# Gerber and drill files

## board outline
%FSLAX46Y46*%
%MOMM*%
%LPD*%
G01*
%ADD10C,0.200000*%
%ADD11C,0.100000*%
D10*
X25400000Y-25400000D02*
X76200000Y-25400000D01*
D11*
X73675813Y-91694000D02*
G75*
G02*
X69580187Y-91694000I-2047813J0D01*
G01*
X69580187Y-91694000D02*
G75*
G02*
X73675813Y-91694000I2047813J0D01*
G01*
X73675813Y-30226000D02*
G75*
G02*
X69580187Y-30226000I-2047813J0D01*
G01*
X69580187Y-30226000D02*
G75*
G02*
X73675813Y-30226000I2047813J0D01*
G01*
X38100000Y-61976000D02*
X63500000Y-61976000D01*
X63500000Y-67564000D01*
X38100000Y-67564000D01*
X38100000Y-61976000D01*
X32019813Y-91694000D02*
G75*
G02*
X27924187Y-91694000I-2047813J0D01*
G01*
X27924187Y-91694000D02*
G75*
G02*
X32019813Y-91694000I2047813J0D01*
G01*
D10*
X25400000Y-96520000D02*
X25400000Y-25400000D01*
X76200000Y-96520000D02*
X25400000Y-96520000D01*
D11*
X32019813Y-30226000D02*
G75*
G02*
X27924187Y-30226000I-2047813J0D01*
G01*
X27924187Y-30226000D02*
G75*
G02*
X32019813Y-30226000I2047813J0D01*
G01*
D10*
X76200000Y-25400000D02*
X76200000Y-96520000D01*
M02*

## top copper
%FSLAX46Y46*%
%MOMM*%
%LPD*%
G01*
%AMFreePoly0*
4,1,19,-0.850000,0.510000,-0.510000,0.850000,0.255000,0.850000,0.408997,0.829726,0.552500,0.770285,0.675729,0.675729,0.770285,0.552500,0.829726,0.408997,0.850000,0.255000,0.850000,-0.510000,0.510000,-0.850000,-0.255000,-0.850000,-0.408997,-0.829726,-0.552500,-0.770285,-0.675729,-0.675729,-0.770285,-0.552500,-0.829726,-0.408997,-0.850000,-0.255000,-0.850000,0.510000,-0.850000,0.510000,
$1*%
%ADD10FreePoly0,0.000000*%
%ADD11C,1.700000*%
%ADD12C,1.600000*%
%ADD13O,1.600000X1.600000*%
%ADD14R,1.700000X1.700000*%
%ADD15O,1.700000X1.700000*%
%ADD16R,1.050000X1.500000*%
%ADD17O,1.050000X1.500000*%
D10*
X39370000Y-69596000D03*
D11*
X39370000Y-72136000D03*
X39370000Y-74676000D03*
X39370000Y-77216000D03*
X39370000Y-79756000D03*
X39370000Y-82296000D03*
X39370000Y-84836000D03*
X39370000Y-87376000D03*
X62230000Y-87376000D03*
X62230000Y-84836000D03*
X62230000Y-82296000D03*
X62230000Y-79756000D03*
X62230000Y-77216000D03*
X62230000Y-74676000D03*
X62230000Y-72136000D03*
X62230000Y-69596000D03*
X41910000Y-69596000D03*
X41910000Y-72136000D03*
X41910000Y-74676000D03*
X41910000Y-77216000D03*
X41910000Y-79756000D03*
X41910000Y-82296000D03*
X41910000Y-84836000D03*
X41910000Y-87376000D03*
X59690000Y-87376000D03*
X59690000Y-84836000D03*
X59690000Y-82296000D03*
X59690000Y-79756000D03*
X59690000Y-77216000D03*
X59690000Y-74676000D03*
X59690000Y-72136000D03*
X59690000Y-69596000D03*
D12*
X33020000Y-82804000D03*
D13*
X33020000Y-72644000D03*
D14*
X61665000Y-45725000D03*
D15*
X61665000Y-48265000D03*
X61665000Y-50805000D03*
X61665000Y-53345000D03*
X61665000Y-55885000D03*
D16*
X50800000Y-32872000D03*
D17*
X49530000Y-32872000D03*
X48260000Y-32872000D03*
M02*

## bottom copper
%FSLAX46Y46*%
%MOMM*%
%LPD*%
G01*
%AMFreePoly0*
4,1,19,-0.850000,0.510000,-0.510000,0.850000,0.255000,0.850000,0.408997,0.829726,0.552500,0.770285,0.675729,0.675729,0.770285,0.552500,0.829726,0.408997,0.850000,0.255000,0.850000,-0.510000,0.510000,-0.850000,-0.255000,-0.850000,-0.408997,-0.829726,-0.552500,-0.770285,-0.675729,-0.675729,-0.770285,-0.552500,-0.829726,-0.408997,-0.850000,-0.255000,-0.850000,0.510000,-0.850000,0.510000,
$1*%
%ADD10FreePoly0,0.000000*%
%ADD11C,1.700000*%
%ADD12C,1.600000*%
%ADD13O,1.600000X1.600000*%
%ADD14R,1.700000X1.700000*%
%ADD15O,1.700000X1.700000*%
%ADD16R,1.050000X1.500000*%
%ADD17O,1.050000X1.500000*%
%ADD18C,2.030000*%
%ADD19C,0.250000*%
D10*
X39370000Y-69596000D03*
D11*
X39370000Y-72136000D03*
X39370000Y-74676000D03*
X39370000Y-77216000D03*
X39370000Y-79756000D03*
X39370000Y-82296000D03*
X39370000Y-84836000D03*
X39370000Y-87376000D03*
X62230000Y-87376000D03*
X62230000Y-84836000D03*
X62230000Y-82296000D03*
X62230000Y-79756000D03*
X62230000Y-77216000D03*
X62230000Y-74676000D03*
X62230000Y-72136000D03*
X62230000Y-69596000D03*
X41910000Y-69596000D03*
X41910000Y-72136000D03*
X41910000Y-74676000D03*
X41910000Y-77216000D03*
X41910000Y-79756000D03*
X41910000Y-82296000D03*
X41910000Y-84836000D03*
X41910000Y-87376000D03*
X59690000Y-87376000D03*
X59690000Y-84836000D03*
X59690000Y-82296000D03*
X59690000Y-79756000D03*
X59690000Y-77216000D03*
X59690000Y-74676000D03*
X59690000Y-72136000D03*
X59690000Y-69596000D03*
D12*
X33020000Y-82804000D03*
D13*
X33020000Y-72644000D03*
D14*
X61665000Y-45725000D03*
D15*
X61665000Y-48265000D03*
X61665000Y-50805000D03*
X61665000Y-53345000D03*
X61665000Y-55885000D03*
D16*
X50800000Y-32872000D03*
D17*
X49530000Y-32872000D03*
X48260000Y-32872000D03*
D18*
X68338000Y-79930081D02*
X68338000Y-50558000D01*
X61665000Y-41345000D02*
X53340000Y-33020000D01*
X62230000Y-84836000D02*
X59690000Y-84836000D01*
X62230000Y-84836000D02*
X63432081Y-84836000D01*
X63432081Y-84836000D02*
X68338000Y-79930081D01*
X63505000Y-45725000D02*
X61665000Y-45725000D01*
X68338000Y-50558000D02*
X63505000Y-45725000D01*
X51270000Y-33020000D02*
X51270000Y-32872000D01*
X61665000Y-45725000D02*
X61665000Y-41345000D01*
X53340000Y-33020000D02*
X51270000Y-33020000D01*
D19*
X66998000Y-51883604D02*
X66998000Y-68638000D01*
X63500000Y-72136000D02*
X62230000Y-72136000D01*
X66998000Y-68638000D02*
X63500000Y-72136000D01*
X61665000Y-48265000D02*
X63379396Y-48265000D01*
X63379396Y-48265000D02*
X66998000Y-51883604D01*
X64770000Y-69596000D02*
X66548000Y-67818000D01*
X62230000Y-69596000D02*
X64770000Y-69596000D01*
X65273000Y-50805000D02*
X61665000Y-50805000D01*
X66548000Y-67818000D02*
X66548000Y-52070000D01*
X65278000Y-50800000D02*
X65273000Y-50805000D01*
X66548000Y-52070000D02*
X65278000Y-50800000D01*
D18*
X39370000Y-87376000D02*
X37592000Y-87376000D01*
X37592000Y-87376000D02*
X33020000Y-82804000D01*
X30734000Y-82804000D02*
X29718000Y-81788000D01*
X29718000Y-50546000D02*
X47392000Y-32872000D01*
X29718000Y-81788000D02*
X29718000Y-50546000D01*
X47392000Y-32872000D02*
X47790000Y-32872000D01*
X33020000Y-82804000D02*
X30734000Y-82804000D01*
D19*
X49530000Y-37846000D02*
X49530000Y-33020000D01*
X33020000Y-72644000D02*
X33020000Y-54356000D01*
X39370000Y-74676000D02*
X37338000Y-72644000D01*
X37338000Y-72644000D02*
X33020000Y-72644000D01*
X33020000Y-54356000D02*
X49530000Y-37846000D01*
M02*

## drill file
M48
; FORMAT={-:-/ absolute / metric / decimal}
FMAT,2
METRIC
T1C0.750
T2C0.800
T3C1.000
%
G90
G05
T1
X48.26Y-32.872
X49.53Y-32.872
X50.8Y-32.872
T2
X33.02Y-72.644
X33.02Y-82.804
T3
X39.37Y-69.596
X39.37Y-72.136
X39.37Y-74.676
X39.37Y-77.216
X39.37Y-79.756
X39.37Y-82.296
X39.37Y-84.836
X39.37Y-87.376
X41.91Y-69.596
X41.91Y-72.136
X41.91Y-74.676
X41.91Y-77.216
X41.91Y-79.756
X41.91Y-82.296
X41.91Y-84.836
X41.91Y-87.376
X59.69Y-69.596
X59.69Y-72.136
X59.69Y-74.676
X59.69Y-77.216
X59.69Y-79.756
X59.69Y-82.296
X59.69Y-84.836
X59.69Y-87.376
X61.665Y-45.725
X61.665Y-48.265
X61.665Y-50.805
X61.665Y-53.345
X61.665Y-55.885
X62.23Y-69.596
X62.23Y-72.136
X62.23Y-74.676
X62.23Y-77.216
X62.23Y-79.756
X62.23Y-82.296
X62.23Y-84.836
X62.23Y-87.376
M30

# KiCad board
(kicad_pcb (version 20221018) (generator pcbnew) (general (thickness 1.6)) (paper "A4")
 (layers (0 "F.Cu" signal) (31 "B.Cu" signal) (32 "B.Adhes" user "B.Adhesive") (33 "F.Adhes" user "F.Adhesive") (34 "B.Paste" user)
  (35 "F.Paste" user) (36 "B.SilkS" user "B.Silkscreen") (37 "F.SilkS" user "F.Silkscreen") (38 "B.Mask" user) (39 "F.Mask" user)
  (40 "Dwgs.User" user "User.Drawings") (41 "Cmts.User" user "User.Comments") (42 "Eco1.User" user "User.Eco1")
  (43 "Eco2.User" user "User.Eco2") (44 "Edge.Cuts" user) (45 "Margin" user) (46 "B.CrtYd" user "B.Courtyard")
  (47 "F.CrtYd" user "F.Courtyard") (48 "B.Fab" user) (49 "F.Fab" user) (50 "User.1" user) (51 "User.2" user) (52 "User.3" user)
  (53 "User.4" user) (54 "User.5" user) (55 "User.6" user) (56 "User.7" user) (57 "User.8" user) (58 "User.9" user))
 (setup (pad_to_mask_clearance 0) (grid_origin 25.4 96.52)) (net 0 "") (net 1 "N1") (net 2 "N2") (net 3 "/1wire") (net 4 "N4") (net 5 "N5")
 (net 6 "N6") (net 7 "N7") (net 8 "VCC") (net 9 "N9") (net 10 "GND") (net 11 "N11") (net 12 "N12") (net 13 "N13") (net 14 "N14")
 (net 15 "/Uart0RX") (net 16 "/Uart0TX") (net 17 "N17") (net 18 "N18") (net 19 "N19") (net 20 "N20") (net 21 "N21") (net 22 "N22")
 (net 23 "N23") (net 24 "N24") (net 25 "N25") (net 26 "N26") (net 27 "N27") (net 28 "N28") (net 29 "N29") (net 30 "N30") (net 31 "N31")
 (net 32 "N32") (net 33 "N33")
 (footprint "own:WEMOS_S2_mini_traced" (layer "F.Cu") (at 39.37 69.596)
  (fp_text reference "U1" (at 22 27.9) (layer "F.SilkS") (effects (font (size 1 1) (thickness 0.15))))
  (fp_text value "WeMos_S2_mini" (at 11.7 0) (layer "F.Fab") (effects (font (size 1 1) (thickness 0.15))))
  (pad "1" thru_hole roundrect (at 0 0) (size 1.7 1.7) (drill 1) (layers "*.Cu" "*.Mask") (roundrect_rratio 0.35) (chamfer_ratio 0.2)
   (chamfer top_left bottom_right) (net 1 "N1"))
  (pad "2" thru_hole circle (at 0 2.54) (size 1.7 1.7) (drill 1) (layers "*.Cu" "*.Mask") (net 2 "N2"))
  (pad "3" thru_hole circle (at 0 5.08) (size 1.7 1.7) (drill 1) (layers "*.Cu" "*.Mask") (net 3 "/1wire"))
  (pad "4" thru_hole circle (at 0 7.62) (size 1.7 1.7) (drill 1) (layers "*.Cu" "*.Mask") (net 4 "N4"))
  (pad "5" thru_hole circle (at 0 10.16) (size 1.7 1.7) (drill 1) (layers "*.Cu" "*.Mask") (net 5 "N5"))
  (pad "6" thru_hole circle (at 0 12.7) (size 1.7 1.7) (drill 1) (layers "*.Cu" "*.Mask") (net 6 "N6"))
  (pad "7" thru_hole circle (at 0 15.24) (size 1.7 1.7) (drill 1) (layers "*.Cu" "*.Mask") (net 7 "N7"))
  (pad "8" thru_hole circle (at 0 17.78) (size 1.7 1.7) (drill 1) (layers "*.Cu" "*.Mask") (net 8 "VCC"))
  (pad "9" thru_hole circle (at 22.86 17.78) (size 1.7 1.7) (drill 1) (layers "*.Cu" "*.Mask") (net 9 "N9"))
  (pad "10" thru_hole circle (at 22.86 15.24) (size 1.7 1.7) (drill 1) (layers "*.Cu" "*.Mask") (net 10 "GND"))
  (pad "11" thru_hole circle (at 22.86 12.7) (size 1.7 1.7) (drill 1) (layers "*.Cu" "*.Mask") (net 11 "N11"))
  (pad "12" thru_hole circle (at 22.86 10.16) (size 1.7 1.7) (drill 1) (layers "*.Cu" "*.Mask") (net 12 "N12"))
  (pad "13" thru_hole circle (at 22.86 7.62) (size 1.7 1.7) (drill 1) (layers "*.Cu" "*.Mask") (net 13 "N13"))
  (pad "14" thru_hole circle (at 22.86 5.08) (size 1.7 1.7) (drill 1) (layers "*.Cu" "*.Mask") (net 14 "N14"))
  (pad "15" thru_hole circle (at 22.86 2.54) (size 1.7 1.7) (drill 1) (layers "*.Cu" "*.Mask") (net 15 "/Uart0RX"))
  (pad "16" thru_hole circle (at 22.86 0) (size 1.7 1.7) (drill 1) (layers "*.Cu" "*.Mask") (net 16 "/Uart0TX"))
  (pad "17" thru_hole circle (at 2.54 0) (size 1.7 1.7) (drill 1) (layers "*.Cu" "*.Mask") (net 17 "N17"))
  (pad "18" thru_hole circle (at 2.54 2.54) (size 1.7 1.7) (drill 1) (layers "*.Cu" "*.Mask") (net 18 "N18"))
  (pad "19" thru_hole circle (at 2.54 5.08) (size 1.7 1.7) (drill 1) (layers "*.Cu" "*.Mask") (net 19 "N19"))
  (pad "20" thru_hole circle (at 2.54 7.62) (size 1.7 1.7) (drill 1) (layers "*.Cu" "*.Mask") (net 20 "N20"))
  (pad "21" thru_hole circle (at 2.54 10.16) (size 1.7 1.7) (drill 1) (layers "*.Cu" "*.Mask") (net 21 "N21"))
  (pad "22" thru_hole circle (at 2.54 12.7) (size 1.7 1.7) (drill 1) (layers "*.Cu" "*.Mask") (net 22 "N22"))
  (pad "23" thru_hole circle (at 2.54 15.24) (size 1.7 1.7) (drill 1) (layers "*.Cu" "*.Mask") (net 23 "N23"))
  (pad "24" thru_hole circle (at 2.54 17.78) (size 1.7 1.7) (drill 1) (layers "*.Cu" "*.Mask") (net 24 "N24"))
  (pad "25" thru_hole circle (at 20.32 17.78) (size 1.7 1.7) (drill 1) (layers "*.Cu" "*.Mask") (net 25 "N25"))
  (pad "26" thru_hole circle (at 20.32 15.24) (size 1.7 1.7) (drill 1) (layers "*.Cu" "*.Mask") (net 10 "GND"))
  (pad "27" thru_hole circle (at 20.32 12.7) (size 1.7 1.7) (drill 1) (layers "*.Cu" "*.Mask") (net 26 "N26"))
  (pad "28" thru_hole circle (at 20.32 10.16) (size 1.7 1.7) (drill 1) (layers "*.Cu" "*.Mask") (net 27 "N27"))
  (pad "29" thru_hole circle (at 20.32 7.62) (size 1.7 1.7) (drill 1) (layers "*.Cu" "*.Mask") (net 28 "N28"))
  (pad "30" thru_hole circle (at 20.32 5.08) (size 1.7 1.7) (drill 1) (layers "*.Cu" "*.Mask") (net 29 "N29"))
  (pad "31" thru_hole circle (at 20.32 2.54) (size 1.7 1.7) (drill 1) (layers "*.Cu" "*.Mask") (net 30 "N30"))
  (pad "32" thru_hole circle (at 20.32 0) (size 1.7 1.7) (drill 1) (layers "*.Cu" "*.Mask") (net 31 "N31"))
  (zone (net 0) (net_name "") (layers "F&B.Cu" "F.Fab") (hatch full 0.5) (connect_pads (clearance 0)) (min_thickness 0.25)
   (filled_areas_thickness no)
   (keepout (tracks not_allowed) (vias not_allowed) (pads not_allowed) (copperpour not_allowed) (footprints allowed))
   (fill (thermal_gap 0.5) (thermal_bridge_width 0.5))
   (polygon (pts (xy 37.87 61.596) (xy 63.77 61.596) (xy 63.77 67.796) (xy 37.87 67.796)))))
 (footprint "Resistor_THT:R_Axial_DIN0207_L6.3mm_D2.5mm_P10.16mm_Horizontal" (layer "F.Cu") (at 33.02 82.804 90)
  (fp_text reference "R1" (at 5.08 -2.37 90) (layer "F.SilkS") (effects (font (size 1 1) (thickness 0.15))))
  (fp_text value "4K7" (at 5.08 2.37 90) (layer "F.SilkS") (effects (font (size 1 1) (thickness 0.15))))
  (pad "1" thru_hole circle (at 0 0 90) (size 1.6 1.6) (drill 0.8) (layers "*.Cu" "*.Mask") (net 8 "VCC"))
  (pad "2" thru_hole oval (at 10.16 0 90) (size 1.6 1.6) (drill 0.8) (layers "*.Cu" "*.Mask") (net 3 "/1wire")))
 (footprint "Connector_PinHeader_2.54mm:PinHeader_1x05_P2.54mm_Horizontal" (layer "F.Cu") (at 61.665 45.725)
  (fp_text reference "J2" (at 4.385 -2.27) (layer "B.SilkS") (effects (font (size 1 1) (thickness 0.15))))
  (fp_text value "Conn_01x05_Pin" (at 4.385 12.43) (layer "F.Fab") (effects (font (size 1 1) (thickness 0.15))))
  (pad "1" thru_hole rect (at 0 0) (size 1.7 1.7) (drill 1) (layers "*.Cu" "*.Mask") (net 10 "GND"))
  (pad "2" thru_hole oval (at 0 2.54) (size 1.7 1.7) (drill 1) (layers "*.Cu" "*.Mask") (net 15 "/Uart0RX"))
  (pad "3" thru_hole oval (at 0 5.08) (size 1.7 1.7) (drill 1) (layers "*.Cu" "*.Mask") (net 16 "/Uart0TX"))
  (pad "4" thru_hole oval (at 0 7.62) (size 1.7 1.7) (drill 1) (layers "*.Cu" "*.Mask") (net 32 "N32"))
  (pad "5" thru_hole oval (at 0 10.16) (size 1.7 1.7) (drill 1) (layers "*.Cu" "*.Mask") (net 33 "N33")))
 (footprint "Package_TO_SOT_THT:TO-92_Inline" (layer "B.Cu") (at 50.8 32.872 180)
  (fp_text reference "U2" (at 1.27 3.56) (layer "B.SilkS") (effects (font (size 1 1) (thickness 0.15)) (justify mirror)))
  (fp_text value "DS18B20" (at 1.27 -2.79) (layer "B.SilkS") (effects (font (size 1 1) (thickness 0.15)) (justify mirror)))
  (pad "1" thru_hole rect (at 0 0 180) (size 1.05 1.5) (drill 0.75) (layers "*.Cu" "*.Mask") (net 10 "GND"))
  (pad "2" thru_hole oval (at 1.27 0 180) (size 1.05 1.5) (drill 0.75) (layers "*.Cu" "*.Mask") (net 3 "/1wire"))
  (pad "3" thru_hole oval (at 2.54 0 180) (size 1.05 1.5) (drill 0.75) (layers "*.Cu" "*.Mask") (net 8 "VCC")))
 (gr_line (start 25.4 25.4) (end 76.2 25.4) (stroke (width 0.2) (type default)) (layer "Edge.Cuts"))
 (gr_circle (center 71.628 91.694) (end 72.644 93.472) (stroke (width 0.1) (type default)) (fill none) (layer "Edge.Cuts"))
 (gr_circle (center 71.628 30.226) (end 72.644 32.004) (stroke (width 0.1) (type default)) (fill none) (layer "Edge.Cuts"))
 (gr_rect (start 38.1 61.976) (end 63.5 67.564) (stroke (width 0.1) (type default)) (fill none) (layer "Edge.Cuts"))
 (gr_circle (center 29.972 91.694) (end 30.988 93.472) (stroke (width 0.1) (type default)) (fill none) (layer "Edge.Cuts"))
 (gr_line (start 25.4 96.52) (end 25.4 25.4) (stroke (width 0.2) (type default)) (layer "Edge.Cuts"))
 (gr_line (start 76.2 96.52) (end 25.4 96.52) (stroke (width 0.2) (type default)) (layer "Edge.Cuts"))
 (gr_circle (center 29.972 30.226) (end 30.988 32.004) (stroke (width 0.1) (type default)) (fill none) (layer "Edge.Cuts"))
 (gr_line (start 76.2 25.4) (end 76.2 96.52) (stroke (width 0.2) (type default)) (layer "Edge.Cuts"))
 (segment (start 68.338 79.930081) (end 68.338 50.558) (width 2.03) (layer "B.Cu") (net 10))
 (segment (start 61.665 41.345) (end 53.34 33.02) (width 2.03) (layer "B.Cu") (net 10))
 (segment (start 62.23 84.836) (end 59.69 84.836) (width 2.03) (layer "B.Cu") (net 10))
 (segment (start 62.23 84.836) (end 63.432081 84.836) (width 2.03) (layer "B.Cu") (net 10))
 (segment (start 63.432081 84.836) (end 68.338 79.930081) (width 2.03) (layer "B.Cu") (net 10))
 (segment (start 63.505 45.725) (end 61.665 45.725) (width 2.03) (layer "B.Cu") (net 10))
 (segment (start 68.338 50.558) (end 63.505 45.725) (width 2.03) (layer "B.Cu") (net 10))
 (segment (start 51.27 33.02) (end 51.27 32.872) (width 2.03) (layer "B.Cu") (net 10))
 (segment (start 61.665 45.725) (end 61.665 41.345) (width 2.03) (layer "B.Cu") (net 10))
 (segment (start 53.34 33.02) (end 51.27 33.02) (width 2.03) (layer "B.Cu") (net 10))
 (segment (start 66.998 51.883604) (end 66.998 68.638) (width 0.25) (layer "B.Cu") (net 15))
 (segment (start 63.5 72.136) (end 62.23 72.136) (width 0.25) (layer "B.Cu") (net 15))
 (segment (start 66.998 68.638) (end 63.5 72.136) (width 0.25) (layer "B.Cu") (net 15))
 (segment (start 61.665 48.265) (end 63.379396 48.265) (width 0.25) (layer "B.Cu") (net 15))
 (segment (start 63.379396 48.265) (end 66.998 51.883604) (width 0.25) (layer "B.Cu") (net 15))
 (segment (start 64.77 69.596) (end 66.548 67.818) (width 0.25) (layer "B.Cu") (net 16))
 (segment (start 62.23 69.596) (end 64.77 69.596) (width 0.25) (layer "B.Cu") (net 16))
 (segment (start 65.273 50.805) (end 61.665 50.805) (width 0.25) (layer "B.Cu") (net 16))
 (segment (start 66.548 67.818) (end 66.548 52.07) (width 0.25) (layer "B.Cu") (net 16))
 (segment (start 65.278 50.8) (end 65.273 50.805) (width 0.25) (layer "B.Cu") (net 16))
 (segment (start 66.548 52.07) (end 65.278 50.8) (width 0.25) (layer "B.Cu") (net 16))
 (segment (start 39.37 87.376) (end 37.592 87.376) (width 2.03) (layer "B.Cu") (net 8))
 (segment (start 37.592 87.376) (end 33.02 82.804) (width 2.03) (layer "B.Cu") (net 8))
 (segment (start 30.734 82.804) (end 29.718 81.788) (width 2.03) (layer "B.Cu") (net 8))
 (segment (start 29.718 50.546) (end 47.392 32.872) (width 2.03) (layer "B.Cu") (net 8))
 (segment (start 29.718 81.788) (end 29.718 50.546) (width 2.03) (layer "B.Cu") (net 8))
 (segment (start 47.392 32.872) (end 47.79 32.872) (width 2.03) (layer "B.Cu") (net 8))
 (segment (start 33.02 82.804) (end 30.734 82.804) (width 2.03) (layer "B.Cu") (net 8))
 (segment (start 49.53 37.846) (end 49.53 33.02) (width 0.25) (layer "B.Cu") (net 3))
 (segment (start 33.02 72.644) (end 33.02 54.356) (width 0.25) (layer "B.Cu") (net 3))
 (segment (start 39.37 74.676) (end 37.338 72.644) (width 0.25) (layer "B.Cu") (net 3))
 (segment (start 37.338 72.644) (end 33.02 72.644) (width 0.25) (layer "B.Cu") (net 3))
 (segment (start 33.02 54.356) (end 49.53 37.846) (width 0.25) (layer "B.Cu") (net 3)))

